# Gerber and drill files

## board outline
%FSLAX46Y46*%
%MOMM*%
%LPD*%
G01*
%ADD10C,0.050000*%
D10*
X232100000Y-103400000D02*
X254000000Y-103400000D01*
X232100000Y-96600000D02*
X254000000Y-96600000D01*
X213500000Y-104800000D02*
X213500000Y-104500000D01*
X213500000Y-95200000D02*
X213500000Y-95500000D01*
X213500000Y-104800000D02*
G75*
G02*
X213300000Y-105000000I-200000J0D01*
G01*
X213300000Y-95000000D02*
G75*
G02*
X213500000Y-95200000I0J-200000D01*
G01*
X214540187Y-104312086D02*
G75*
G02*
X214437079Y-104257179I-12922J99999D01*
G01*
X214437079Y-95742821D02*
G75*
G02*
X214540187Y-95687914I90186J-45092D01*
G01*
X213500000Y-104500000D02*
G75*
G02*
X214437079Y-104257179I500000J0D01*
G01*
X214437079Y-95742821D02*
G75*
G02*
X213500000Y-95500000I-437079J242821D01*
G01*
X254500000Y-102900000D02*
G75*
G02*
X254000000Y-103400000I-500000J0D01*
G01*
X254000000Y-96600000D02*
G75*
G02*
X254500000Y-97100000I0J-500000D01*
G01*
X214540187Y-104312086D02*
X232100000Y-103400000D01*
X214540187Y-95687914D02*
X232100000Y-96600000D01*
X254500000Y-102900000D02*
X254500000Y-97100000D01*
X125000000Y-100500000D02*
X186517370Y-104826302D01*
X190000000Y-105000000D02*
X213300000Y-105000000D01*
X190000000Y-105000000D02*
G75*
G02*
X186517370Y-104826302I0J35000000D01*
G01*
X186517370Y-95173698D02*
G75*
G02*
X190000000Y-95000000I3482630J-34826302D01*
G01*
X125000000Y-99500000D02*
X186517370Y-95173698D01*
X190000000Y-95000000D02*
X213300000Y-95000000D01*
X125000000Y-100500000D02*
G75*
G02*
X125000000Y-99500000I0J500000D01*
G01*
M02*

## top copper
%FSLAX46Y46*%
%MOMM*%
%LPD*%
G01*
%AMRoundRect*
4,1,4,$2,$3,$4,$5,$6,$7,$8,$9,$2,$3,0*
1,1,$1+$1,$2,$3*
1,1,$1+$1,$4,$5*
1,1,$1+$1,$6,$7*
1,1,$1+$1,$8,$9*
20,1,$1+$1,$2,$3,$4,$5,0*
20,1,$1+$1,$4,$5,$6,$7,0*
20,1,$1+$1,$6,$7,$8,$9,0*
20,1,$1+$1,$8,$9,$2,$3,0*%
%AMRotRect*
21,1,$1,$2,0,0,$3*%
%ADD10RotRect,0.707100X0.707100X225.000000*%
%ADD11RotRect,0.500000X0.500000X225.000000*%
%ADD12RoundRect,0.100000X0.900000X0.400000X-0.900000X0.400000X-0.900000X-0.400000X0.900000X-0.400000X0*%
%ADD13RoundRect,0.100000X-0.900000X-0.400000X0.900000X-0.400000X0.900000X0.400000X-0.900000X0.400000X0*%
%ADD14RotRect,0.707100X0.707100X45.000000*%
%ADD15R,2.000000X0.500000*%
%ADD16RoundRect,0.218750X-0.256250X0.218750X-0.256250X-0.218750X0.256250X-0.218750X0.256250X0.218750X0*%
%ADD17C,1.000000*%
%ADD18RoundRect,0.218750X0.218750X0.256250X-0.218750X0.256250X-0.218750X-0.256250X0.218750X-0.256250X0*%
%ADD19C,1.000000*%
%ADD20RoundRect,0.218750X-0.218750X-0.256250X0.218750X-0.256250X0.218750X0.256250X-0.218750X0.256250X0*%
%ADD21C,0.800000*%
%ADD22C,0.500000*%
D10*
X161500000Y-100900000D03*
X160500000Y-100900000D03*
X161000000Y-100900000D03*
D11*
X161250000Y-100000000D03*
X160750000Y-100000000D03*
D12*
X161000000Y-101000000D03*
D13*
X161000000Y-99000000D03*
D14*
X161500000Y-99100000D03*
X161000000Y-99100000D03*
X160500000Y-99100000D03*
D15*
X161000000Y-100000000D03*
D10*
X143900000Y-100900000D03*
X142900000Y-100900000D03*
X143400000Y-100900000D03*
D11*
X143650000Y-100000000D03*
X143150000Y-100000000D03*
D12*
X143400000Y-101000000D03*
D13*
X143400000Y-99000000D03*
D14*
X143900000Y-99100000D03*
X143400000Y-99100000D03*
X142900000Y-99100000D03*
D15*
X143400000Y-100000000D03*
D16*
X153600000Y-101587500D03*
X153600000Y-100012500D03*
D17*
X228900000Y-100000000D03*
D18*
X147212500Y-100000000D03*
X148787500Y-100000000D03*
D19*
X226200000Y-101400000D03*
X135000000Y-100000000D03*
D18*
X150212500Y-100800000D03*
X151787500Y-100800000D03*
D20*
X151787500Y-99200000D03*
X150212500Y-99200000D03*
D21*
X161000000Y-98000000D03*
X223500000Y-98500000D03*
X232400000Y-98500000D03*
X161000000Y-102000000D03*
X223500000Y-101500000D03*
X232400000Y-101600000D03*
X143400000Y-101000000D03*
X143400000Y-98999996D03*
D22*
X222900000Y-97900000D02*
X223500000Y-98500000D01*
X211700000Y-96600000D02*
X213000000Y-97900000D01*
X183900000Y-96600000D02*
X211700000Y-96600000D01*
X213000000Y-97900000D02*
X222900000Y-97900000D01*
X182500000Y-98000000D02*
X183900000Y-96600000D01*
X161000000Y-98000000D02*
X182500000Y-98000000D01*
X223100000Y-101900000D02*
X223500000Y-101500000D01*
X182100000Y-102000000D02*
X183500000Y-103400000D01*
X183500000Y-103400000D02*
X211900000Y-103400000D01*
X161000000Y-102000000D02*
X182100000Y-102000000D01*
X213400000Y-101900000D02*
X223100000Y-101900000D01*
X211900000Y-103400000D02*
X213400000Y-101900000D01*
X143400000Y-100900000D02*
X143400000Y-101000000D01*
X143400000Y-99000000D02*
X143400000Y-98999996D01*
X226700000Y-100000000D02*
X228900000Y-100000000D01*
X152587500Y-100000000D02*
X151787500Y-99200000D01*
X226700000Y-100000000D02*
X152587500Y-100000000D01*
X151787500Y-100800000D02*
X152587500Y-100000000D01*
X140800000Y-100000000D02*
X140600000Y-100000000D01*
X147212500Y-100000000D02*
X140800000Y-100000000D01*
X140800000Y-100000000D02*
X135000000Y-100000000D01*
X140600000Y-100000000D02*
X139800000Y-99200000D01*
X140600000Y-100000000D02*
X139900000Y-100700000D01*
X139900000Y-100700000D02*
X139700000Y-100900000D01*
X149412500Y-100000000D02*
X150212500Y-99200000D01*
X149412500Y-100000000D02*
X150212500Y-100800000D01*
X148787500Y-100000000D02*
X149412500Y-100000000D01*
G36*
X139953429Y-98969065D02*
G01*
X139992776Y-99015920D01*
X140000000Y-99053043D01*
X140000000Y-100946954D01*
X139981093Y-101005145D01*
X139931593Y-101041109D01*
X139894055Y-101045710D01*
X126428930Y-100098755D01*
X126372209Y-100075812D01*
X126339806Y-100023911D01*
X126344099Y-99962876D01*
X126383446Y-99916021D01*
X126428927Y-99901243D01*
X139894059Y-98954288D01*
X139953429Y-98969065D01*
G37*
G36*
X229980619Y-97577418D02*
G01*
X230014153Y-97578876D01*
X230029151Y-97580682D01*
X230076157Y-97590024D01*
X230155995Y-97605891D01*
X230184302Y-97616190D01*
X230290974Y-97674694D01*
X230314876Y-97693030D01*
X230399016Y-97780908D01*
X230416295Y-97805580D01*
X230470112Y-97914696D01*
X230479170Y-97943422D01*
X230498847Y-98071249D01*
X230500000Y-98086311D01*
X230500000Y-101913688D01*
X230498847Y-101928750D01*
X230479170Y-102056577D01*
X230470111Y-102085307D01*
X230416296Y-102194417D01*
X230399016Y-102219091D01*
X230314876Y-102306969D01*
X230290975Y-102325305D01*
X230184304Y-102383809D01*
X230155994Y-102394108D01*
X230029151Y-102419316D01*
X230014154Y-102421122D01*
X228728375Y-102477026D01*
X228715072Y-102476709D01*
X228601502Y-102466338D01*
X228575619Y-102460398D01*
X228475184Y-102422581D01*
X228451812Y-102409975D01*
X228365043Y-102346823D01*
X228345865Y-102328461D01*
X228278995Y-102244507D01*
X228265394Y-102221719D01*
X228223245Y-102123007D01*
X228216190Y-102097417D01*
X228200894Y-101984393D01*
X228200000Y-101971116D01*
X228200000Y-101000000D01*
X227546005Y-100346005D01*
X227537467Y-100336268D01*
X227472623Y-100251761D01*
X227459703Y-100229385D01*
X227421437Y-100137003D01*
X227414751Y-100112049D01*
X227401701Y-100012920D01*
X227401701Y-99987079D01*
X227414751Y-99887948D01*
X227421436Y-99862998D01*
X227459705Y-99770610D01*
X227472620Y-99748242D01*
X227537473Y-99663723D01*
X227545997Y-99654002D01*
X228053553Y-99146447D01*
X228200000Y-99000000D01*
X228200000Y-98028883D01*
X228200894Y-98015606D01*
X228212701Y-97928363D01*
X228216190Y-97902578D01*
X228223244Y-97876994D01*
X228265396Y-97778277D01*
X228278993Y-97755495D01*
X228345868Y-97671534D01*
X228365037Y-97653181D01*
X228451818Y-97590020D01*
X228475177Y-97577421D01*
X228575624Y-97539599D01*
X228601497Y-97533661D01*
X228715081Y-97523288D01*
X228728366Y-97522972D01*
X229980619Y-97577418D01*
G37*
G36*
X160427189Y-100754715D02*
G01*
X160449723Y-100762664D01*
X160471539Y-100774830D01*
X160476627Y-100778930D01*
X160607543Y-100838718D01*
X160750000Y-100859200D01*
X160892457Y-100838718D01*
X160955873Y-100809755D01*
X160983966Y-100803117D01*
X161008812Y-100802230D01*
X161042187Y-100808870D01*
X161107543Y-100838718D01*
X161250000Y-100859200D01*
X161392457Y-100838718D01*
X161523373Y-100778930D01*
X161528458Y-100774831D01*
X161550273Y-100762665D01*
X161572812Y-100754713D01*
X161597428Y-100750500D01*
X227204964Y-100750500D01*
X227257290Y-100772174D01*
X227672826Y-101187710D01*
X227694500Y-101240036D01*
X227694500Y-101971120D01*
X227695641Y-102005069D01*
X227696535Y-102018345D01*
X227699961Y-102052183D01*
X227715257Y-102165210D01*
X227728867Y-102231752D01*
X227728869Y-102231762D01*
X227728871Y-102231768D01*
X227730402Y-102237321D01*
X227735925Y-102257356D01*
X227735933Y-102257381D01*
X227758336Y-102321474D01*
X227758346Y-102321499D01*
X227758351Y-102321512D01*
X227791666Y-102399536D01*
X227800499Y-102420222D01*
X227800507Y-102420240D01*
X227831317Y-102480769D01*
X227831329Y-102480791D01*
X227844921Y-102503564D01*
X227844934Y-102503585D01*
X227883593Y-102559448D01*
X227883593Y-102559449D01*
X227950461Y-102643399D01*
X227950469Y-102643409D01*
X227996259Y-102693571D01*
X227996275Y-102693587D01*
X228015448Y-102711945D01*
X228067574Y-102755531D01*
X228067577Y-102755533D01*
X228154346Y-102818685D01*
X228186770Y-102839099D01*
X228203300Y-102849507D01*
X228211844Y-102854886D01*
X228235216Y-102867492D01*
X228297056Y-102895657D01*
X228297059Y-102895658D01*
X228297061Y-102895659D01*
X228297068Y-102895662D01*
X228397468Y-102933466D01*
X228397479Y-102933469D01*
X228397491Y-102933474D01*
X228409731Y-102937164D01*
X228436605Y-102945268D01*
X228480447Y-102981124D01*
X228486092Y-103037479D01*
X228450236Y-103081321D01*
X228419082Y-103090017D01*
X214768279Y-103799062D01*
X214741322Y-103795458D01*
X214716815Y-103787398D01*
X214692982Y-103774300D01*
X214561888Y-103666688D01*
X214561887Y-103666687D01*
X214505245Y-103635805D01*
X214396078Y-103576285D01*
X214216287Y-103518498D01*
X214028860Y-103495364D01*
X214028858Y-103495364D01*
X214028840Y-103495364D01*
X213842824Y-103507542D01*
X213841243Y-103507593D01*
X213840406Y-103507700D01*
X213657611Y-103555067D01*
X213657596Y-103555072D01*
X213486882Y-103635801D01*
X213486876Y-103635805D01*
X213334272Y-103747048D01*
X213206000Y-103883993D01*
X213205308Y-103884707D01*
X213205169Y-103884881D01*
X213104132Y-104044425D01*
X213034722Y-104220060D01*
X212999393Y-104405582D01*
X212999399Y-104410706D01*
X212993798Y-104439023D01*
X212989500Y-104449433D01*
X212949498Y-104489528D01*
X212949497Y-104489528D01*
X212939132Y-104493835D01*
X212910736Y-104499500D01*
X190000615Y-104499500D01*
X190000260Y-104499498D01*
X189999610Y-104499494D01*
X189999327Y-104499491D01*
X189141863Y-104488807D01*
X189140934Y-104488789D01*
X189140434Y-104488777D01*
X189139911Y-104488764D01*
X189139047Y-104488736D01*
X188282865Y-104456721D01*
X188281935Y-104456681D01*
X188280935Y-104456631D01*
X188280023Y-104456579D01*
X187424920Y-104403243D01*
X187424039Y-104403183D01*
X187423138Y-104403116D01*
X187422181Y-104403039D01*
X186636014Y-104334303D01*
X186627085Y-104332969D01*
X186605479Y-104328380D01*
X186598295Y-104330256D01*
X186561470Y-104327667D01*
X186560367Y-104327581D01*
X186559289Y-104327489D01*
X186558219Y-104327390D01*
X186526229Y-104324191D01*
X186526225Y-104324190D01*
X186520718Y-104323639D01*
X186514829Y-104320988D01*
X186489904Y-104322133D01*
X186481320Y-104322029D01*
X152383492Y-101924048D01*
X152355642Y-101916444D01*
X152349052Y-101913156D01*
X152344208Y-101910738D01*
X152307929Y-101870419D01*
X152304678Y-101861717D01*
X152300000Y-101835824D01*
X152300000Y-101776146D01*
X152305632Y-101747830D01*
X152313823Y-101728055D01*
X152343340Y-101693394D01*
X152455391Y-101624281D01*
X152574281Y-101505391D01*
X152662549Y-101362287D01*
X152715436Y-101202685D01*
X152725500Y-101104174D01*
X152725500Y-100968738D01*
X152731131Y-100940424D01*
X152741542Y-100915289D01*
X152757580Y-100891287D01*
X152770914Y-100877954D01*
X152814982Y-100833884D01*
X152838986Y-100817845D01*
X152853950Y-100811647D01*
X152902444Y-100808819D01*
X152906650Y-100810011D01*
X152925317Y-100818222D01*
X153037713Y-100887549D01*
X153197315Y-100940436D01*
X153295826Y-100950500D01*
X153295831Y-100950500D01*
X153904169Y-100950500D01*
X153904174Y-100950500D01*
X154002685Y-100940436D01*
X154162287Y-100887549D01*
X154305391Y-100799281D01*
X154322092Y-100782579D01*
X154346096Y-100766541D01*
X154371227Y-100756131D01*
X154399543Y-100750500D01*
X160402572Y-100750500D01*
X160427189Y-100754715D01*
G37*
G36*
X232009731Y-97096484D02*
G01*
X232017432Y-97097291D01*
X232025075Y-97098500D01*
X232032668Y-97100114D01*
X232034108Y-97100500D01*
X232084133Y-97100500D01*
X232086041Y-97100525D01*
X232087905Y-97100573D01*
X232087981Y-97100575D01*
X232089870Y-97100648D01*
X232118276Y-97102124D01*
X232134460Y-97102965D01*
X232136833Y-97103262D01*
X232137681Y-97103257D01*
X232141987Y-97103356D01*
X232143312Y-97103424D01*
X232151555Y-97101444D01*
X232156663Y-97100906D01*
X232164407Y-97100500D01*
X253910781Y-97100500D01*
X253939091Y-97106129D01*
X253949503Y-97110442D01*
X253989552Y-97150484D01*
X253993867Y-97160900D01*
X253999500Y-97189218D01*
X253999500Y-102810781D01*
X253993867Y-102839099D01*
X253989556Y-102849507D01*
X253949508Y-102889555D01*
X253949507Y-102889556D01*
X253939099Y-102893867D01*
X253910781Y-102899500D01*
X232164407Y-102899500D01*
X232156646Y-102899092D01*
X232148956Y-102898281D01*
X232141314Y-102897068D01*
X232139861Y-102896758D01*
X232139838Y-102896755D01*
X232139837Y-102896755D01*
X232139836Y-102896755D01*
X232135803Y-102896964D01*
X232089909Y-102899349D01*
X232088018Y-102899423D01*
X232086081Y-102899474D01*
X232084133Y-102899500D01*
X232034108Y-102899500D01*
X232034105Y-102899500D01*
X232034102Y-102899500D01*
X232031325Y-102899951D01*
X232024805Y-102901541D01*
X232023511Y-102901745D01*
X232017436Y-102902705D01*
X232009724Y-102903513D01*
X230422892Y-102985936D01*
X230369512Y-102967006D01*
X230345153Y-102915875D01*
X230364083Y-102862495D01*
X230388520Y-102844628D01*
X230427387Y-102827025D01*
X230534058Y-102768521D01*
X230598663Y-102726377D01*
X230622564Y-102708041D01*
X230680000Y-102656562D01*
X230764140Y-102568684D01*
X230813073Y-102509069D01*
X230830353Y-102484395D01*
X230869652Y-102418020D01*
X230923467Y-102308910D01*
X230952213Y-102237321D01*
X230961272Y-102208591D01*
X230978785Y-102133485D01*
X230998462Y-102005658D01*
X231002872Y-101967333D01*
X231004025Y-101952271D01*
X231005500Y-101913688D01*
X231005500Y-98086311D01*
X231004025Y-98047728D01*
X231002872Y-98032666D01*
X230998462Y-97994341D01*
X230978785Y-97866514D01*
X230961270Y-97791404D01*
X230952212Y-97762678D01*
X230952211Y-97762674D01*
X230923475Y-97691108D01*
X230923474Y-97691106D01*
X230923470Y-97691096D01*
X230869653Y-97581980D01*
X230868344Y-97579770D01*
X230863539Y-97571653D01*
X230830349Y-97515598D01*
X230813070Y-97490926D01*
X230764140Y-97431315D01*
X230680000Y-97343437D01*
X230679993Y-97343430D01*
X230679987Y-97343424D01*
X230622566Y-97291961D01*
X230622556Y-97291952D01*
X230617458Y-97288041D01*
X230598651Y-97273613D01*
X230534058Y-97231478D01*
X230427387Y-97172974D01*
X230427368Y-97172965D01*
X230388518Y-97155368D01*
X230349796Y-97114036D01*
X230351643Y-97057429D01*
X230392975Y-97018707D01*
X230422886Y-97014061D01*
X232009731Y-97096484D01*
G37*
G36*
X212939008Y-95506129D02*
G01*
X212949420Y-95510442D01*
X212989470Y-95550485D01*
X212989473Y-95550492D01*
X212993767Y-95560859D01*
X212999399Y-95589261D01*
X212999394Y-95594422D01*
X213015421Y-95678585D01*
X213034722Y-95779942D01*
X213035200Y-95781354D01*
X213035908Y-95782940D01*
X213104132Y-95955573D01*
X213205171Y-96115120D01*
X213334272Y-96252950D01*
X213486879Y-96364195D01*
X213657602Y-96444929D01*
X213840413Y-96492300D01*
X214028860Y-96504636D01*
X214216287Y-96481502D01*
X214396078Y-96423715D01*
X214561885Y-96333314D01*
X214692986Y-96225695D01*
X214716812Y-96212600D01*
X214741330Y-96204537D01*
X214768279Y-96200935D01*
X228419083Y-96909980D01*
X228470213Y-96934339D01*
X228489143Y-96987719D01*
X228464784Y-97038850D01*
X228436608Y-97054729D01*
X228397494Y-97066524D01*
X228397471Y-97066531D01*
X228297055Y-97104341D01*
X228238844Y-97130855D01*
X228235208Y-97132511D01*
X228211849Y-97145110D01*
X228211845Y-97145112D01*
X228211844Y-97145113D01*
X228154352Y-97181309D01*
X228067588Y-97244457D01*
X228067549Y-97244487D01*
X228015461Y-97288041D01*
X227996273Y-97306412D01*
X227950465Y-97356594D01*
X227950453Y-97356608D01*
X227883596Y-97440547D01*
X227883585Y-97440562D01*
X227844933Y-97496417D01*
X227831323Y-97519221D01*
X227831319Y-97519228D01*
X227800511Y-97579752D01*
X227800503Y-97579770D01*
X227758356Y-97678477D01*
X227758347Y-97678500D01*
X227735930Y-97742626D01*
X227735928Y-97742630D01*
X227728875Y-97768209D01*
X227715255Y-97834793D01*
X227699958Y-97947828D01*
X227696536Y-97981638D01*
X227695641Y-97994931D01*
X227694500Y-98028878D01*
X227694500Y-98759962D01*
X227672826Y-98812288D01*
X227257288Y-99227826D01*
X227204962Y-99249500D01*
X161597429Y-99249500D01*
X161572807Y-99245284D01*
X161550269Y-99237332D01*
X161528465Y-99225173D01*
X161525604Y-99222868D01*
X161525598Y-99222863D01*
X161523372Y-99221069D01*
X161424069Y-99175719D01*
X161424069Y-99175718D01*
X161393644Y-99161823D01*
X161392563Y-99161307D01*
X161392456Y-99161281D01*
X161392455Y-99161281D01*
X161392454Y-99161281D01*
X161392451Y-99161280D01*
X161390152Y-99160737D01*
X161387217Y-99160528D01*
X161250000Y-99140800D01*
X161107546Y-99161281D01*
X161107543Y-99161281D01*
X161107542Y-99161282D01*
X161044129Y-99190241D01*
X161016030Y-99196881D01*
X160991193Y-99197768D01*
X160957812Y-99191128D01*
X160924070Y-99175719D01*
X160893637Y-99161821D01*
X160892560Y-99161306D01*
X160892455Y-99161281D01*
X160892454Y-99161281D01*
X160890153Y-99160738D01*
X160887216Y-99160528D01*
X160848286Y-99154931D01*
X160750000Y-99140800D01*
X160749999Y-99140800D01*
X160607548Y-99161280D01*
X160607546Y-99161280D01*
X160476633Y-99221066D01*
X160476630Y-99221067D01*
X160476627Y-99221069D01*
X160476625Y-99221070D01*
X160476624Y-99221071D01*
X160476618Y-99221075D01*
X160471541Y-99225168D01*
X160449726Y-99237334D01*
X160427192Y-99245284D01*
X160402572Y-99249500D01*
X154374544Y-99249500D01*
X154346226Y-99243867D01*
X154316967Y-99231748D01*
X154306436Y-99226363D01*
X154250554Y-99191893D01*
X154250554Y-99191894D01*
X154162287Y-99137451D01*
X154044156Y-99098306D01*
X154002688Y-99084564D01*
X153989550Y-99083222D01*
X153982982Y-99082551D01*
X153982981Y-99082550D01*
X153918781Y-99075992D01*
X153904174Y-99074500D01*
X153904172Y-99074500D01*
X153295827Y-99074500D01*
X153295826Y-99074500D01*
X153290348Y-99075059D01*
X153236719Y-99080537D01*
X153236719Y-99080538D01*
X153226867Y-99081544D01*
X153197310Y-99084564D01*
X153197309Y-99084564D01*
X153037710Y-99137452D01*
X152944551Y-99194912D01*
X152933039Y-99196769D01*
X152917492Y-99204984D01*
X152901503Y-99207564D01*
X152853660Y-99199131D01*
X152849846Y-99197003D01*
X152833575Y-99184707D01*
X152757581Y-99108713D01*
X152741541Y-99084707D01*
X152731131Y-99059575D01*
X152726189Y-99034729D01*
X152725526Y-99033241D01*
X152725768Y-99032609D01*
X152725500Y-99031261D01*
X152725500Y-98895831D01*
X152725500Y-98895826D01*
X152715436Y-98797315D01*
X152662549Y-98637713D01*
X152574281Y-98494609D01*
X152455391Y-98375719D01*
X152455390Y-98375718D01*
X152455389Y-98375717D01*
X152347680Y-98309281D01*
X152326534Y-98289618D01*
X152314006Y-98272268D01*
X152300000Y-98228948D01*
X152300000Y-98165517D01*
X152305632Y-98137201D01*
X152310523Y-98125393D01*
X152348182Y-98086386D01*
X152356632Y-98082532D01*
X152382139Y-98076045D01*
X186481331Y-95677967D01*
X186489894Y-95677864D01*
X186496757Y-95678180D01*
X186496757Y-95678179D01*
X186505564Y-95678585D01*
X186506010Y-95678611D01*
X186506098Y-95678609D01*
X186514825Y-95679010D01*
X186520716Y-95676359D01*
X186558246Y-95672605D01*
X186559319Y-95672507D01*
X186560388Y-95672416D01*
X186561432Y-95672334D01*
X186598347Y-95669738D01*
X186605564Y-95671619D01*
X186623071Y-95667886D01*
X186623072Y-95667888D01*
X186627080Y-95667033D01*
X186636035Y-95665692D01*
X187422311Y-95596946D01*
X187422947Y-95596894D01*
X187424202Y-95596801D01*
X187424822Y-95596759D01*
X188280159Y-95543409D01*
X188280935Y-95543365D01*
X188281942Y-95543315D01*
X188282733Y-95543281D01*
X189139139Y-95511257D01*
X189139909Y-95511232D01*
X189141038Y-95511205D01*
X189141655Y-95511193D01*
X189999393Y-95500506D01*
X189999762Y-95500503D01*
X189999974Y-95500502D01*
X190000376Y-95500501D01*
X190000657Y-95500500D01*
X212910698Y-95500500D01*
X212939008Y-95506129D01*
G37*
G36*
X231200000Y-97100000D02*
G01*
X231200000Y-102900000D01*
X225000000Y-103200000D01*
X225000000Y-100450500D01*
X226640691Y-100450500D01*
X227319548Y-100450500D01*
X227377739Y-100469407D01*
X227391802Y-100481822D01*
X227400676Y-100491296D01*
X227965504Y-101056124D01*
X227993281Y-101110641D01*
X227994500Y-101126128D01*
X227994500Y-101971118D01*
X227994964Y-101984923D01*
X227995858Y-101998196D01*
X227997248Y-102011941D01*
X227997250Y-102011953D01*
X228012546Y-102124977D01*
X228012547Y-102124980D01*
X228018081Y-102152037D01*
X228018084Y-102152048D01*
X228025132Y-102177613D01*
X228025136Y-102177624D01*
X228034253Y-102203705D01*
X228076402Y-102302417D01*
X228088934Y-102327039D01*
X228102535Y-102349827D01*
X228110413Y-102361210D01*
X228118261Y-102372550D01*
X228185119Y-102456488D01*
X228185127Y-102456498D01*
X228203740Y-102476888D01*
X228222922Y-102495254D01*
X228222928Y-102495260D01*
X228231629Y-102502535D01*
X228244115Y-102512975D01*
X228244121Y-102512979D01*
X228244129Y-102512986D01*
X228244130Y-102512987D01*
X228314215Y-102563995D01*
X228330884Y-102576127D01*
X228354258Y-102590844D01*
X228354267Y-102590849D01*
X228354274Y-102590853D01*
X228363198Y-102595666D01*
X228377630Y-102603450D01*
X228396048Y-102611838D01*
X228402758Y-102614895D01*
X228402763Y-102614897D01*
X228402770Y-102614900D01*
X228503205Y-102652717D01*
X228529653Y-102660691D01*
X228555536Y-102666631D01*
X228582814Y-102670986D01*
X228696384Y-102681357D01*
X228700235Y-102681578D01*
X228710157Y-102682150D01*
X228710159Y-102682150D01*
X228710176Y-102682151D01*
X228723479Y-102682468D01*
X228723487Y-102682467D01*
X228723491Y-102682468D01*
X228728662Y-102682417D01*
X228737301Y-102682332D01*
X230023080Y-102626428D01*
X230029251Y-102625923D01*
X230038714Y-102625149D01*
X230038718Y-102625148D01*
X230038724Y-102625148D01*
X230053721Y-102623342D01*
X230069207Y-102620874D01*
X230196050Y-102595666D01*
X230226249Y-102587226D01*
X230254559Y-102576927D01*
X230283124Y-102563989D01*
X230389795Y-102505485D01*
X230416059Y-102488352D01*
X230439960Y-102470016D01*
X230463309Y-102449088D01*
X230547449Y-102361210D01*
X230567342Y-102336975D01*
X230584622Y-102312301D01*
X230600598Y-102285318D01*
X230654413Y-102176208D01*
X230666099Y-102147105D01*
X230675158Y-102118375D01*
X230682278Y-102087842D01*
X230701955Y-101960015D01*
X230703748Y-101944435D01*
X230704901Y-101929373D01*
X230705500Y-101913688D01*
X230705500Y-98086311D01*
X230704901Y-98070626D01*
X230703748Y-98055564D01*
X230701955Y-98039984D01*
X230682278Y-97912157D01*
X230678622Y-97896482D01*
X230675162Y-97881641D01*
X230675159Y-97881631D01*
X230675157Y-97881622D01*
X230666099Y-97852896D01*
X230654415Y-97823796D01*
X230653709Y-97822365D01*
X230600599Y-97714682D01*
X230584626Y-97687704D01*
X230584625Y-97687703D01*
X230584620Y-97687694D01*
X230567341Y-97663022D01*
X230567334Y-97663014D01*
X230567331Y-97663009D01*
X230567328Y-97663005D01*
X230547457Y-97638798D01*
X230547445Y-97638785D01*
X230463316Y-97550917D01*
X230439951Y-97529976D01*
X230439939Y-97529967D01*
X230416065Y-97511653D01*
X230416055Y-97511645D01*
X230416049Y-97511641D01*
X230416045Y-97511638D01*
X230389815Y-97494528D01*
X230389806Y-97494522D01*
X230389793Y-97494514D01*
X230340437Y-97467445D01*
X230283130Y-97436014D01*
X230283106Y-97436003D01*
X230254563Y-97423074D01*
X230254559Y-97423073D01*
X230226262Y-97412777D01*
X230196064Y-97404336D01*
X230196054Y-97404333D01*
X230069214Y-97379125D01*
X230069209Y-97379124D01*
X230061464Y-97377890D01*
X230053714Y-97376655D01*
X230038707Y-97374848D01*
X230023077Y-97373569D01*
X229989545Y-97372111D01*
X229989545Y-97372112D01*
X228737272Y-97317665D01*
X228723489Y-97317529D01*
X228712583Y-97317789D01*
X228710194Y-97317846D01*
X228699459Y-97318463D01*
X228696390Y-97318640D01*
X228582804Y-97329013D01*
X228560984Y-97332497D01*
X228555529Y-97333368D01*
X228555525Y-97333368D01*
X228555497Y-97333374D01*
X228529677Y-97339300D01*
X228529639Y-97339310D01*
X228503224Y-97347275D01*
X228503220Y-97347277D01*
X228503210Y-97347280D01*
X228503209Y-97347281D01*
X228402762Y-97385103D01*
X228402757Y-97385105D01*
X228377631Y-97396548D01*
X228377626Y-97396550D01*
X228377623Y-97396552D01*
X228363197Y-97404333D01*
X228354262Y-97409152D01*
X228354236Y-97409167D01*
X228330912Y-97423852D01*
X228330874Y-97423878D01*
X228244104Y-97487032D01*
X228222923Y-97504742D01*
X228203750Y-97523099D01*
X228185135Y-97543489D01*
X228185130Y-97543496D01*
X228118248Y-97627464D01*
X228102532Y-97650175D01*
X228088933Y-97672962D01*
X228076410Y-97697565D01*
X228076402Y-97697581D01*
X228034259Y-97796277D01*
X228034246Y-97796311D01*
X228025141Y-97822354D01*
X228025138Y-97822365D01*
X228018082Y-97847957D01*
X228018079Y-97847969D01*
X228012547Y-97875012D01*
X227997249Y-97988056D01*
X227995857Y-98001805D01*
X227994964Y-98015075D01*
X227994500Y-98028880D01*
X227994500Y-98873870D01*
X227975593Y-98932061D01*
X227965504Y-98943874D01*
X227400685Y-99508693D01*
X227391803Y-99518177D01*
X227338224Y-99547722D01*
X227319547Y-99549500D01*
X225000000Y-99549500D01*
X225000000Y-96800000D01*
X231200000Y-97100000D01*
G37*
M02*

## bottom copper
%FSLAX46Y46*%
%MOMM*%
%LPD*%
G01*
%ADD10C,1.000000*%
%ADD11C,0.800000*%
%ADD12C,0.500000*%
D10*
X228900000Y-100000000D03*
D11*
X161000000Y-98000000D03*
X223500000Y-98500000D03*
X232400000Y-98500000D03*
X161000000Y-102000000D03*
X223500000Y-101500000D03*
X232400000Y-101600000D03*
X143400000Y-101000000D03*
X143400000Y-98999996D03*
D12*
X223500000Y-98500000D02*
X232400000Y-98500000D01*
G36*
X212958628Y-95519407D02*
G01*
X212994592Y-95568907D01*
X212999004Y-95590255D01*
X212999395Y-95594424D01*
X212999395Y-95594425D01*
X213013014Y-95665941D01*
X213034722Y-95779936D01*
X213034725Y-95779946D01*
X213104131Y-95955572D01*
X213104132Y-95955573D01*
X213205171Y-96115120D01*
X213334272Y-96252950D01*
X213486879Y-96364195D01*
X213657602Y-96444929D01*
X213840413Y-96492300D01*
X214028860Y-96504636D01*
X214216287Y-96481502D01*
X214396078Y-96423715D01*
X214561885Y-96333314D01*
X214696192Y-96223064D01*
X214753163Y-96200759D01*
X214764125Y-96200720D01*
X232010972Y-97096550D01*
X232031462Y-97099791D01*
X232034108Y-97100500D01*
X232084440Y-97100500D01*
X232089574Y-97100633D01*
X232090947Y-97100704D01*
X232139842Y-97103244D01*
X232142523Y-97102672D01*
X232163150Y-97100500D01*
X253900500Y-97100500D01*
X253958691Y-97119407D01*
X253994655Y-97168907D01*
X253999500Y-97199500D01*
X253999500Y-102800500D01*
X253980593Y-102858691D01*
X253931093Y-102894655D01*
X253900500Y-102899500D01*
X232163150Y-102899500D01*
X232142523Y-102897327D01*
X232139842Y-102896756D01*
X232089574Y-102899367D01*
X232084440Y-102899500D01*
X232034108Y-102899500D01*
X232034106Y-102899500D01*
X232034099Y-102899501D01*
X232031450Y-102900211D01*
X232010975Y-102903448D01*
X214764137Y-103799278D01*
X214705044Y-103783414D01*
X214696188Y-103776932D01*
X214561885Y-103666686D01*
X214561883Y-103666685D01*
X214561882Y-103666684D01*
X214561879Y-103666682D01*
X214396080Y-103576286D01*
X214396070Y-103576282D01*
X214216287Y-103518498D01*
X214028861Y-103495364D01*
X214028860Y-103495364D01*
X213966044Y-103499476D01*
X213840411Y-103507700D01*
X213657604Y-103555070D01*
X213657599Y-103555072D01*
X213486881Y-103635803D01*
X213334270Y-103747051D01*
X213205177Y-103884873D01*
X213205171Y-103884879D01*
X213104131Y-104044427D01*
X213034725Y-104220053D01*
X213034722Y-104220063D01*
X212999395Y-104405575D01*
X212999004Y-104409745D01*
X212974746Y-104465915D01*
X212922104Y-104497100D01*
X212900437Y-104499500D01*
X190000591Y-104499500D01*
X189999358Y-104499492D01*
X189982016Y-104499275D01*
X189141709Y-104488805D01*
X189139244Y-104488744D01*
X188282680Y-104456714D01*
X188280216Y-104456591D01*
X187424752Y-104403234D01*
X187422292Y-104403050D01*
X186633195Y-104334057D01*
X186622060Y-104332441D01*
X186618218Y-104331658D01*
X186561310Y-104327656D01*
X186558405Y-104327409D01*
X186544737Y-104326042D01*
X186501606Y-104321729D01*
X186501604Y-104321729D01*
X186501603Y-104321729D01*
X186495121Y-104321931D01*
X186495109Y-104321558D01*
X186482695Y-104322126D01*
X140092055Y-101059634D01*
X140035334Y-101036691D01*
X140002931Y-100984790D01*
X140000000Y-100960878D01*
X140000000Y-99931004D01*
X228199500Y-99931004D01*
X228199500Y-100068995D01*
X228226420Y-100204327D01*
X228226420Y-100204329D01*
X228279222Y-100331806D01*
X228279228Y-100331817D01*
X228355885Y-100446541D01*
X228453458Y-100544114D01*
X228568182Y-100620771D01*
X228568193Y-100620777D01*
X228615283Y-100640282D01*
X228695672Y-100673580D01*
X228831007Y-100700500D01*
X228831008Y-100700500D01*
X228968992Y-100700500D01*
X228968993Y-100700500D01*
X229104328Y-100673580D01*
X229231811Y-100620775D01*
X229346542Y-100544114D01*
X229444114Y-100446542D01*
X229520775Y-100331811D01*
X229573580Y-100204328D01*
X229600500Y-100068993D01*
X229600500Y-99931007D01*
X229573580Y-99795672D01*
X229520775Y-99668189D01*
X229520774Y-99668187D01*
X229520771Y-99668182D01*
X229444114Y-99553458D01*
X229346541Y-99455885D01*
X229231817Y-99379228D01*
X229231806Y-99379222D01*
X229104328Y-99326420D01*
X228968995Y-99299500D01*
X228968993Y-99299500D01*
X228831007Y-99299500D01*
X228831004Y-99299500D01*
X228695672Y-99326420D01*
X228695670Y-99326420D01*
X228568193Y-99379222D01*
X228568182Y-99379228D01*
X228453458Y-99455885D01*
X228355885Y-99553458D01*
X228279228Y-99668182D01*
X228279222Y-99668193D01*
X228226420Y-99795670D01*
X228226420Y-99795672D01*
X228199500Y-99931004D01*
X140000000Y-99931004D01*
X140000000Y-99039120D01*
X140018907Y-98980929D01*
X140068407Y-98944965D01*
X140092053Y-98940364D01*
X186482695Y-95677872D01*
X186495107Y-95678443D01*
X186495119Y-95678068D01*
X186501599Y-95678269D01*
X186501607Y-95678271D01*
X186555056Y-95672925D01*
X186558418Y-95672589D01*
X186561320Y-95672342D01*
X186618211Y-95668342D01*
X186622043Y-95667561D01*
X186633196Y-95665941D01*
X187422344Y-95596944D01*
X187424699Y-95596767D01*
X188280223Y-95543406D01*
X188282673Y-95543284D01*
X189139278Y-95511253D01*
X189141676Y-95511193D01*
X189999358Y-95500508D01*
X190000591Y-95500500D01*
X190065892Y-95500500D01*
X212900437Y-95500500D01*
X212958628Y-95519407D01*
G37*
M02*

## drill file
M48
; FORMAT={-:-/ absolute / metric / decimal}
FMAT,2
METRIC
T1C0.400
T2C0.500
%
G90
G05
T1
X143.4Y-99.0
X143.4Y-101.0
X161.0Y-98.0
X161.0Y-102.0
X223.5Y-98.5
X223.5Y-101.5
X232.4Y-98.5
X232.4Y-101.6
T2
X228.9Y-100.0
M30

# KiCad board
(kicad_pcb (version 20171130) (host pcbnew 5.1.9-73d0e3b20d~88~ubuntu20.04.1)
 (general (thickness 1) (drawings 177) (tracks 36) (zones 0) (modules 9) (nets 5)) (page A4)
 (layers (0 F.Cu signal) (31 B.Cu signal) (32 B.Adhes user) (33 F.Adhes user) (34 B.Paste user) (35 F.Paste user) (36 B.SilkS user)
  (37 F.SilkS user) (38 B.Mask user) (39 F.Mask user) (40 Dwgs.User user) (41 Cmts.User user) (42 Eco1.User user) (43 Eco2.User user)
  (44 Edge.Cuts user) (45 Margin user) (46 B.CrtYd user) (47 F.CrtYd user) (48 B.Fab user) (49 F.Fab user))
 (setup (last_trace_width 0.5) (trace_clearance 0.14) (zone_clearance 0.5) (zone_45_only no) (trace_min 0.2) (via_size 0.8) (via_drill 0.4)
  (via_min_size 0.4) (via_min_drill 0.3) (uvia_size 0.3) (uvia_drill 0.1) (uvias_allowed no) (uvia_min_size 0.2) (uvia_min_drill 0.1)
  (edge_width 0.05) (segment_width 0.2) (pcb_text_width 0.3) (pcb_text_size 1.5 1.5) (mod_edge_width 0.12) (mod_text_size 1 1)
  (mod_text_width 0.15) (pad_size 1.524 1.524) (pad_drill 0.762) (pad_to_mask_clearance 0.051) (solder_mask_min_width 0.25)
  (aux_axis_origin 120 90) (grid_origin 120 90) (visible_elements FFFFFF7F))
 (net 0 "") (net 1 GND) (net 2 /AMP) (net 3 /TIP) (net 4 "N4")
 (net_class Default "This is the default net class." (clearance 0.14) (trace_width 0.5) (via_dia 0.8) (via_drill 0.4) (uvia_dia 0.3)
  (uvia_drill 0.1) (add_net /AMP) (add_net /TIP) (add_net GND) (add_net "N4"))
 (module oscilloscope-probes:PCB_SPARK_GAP (layer F.Cu) (at 161 100)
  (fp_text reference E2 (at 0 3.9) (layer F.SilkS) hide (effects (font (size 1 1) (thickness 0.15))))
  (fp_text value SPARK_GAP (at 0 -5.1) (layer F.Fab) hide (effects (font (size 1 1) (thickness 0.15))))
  (pad 2 smd rect (at 0.5 0.9 225) (size 0.7071 0.7071) (layers F.Cu) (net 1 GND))
  (pad 2 smd rect (at -0.5 0.9 225) (size 0.7071 0.7071) (layers F.Cu) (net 1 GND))
  (pad 2 smd rect (at 0 0.9 225) (size 0.7071 0.7071) (layers F.Cu) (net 1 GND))
  (pad 1 smd rect (at 0.25 0 225) (size 0.5 0.5) (layers F.Cu F.Mask) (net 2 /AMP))
  (pad 1 smd rect (at -0.25 0 225) (size 0.5 0.5) (layers F.Cu F.Mask) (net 2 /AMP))
  (pad 2 smd roundrect (at 0 1 180) (size 2 1) (layers F.Cu) (roundrect_rratio 0.1) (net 1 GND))
  (pad 2 smd roundrect (at 0 -1) (size 2 1) (layers F.Cu) (roundrect_rratio 0.1) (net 1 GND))
  (pad 2 smd rect (at 0.5 -0.9 45) (size 0.7071 0.7071) (layers F.Cu) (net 1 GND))
  (pad 2 smd rect (at 0 -0.9 45) (size 0.7071 0.7071) (layers F.Cu) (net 1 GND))
  (pad 2 smd rect (at -0.5 -0.9 45) (size 0.7071 0.7071) (layers F.Cu) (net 1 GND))
  (pad 1 smd rect (at 0 0) (size 2 0.5) (layers F.Cu F.Mask) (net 2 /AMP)))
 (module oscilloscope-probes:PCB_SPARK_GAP (layer F.Cu) (at 143.4 100)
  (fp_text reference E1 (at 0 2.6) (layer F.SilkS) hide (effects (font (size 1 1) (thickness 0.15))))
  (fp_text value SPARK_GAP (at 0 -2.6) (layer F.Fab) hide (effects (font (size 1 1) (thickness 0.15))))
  (pad 2 smd rect (at 0.5 0.9 225) (size 0.7071 0.7071) (layers F.Cu) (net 1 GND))
  (pad 2 smd rect (at -0.5 0.9 225) (size 0.7071 0.7071) (layers F.Cu) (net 1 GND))
  (pad 2 smd rect (at 0 0.9 225) (size 0.7071 0.7071) (layers F.Cu) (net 1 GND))
  (pad 1 smd rect (at 0.25 0 225) (size 0.5 0.5) (layers F.Cu F.Mask) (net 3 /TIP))
  (pad 1 smd rect (at -0.25 0 225) (size 0.5 0.5) (layers F.Cu F.Mask) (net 3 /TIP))
  (pad 2 smd roundrect (at 0 1 180) (size 2 1) (layers F.Cu) (roundrect_rratio 0.1) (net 1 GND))
  (pad 2 smd roundrect (at 0 -1) (size 2 1) (layers F.Cu) (roundrect_rratio 0.1) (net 1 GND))
  (pad 2 smd rect (at 0.5 -0.9 45) (size 0.7071 0.7071) (layers F.Cu) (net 1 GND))
  (pad 2 smd rect (at 0 -0.9 45) (size 0.7071 0.7071) (layers F.Cu) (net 1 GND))
  (pad 2 smd rect (at -0.5 -0.9 45) (size 0.7071 0.7071) (layers F.Cu) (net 1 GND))
  (pad 1 smd rect (at 0 0) (size 2 0.5) (layers F.Cu F.Mask) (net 3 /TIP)))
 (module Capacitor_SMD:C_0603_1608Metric (layer F.Cu) (at 153.6 100.8 270)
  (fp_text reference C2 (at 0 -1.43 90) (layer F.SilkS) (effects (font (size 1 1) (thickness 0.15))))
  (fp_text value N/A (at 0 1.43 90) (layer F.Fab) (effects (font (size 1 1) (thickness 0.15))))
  (pad 2 smd roundrect (at 0.7875 0 270) (size 0.875 0.95) (layers F.Cu F.Paste F.Mask) (roundrect_rratio 0.25) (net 1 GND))
  (pad 1 smd roundrect (at -0.7875 0 270) (size 0.875 0.95) (layers F.Cu F.Paste F.Mask) (roundrect_rratio 0.25) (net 2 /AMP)))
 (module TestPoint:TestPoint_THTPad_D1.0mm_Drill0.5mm (layer F.Cu) (at 228.9 100)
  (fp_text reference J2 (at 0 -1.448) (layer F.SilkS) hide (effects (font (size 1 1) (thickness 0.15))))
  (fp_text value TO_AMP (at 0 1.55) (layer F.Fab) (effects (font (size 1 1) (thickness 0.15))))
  (pad 1 thru_hole circle (at 0 0) (size 1 1) (drill 0.5) (layers *.Cu *.Mask) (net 2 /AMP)))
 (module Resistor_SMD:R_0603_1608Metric (layer F.Cu) (at 148 100 180)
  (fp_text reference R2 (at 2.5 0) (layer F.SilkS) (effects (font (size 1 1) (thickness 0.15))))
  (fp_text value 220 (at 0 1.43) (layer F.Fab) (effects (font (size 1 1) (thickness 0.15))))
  (pad 2 smd roundrect (at 0.7875 0 180) (size 0.875 0.95) (layers F.Cu F.Paste F.Mask) (roundrect_rratio 0.25) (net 3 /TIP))
  (pad 1 smd roundrect (at -0.7875 0 180) (size 0.875 0.95) (layers F.Cu F.Paste F.Mask) (roundrect_rratio 0.25) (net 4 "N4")))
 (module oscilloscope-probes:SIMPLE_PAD (layer F.Cu) (at 226.2 101.4)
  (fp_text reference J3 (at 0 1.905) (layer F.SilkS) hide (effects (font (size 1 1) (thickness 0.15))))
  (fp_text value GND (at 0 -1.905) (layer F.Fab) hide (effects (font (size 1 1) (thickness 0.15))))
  (pad 1 smd circle (at 0 0) (size 1 1) (layers F.Cu F.Mask) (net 1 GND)))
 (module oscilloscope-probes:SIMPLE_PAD (layer F.Cu) (at 135 100)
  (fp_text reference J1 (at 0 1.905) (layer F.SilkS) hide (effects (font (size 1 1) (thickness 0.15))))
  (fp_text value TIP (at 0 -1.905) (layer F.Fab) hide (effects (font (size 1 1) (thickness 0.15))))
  (pad 1 smd circle (at 0 0) (size 1 1) (layers F.Cu F.Mask) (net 3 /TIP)))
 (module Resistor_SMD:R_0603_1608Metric (layer F.Cu) (at 151 100.8 180)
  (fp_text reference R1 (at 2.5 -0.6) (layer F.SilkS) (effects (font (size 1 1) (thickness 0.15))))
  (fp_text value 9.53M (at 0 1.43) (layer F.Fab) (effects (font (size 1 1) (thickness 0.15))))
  (pad 2 smd roundrect (at 0.7875 0 180) (size 0.875 0.95) (layers F.Cu F.Paste F.Mask) (roundrect_rratio 0.25) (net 4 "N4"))
  (pad 1 smd roundrect (at -0.7875 0 180) (size 0.875 0.95) (layers F.Cu F.Paste F.Mask) (roundrect_rratio 0.25) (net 2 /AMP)))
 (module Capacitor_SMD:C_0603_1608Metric (layer F.Cu) (at 151 99.2)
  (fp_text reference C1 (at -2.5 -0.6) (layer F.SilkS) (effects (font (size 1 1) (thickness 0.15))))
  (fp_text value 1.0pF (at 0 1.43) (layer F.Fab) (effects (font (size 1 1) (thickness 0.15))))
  (pad 2 smd roundrect (at 0.7875 0) (size 0.875 0.95) (layers F.Cu F.Paste F.Mask) (roundrect_rratio 0.25) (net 2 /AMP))
  (pad 1 smd roundrect (at -0.7875 0) (size 0.875 0.95) (layers F.Cu F.Paste F.Mask) (roundrect_rratio 0.25) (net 4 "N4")))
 (gr_line (start 232.1 103.4) (end 254 103.4) (layer Edge.Cuts) (width 0.05))
 (gr_line (start 232.1 96.6) (end 254 96.6) (layer Edge.Cuts) (width 0.05))
 (gr_line (start 213.5 104.8) (end 213.5 104.5) (layer Edge.Cuts) (width 0.05))
 (gr_line (start 213.5 95.2) (end 213.5 95.5) (layer Edge.Cuts) (width 0.05))
 (gr_arc (start 213.3 104.8) (end 213.5 104.8) (angle 90) (layer Edge.Cuts) (width 0.05))
 (gr_arc (start 213.3 95.2) (end 213.5 95.2) (angle -90) (layer Edge.Cuts) (width 0.05))
 (gr_arc (start 214.527265 104.212087) (end 214.540187 104.312086) (angle 70.79848966) (layer Edge.Cuts) (width 0.05))
 (gr_arc (start 214.527265 95.787913) (end 214.540187 95.687914) (angle -70.79848966) (layer Edge.Cuts) (width 0.05))
 (gr_arc (start 214 104.5) (end 213.5 104.5) (angle 150.9453959) (layer Edge.Cuts) (width 0.05))
 (gr_arc (start 214 95.5) (end 213.5 95.5) (angle -150.9453959) (layer Edge.Cuts) (width 0.05))
 (gr_arc (start 254 102.9) (end 254 103.4) (angle -90) (layer Edge.Cuts) (width 0.05))
 (gr_arc (start 254 97.1) (end 254.5 97.1) (angle -90) (layer Edge.Cuts) (width 0.05))
 (gr_line (start 214.540187 104.312086) (end 232.1 103.4) (layer Edge.Cuts) (width 0.05))
 (gr_line (start 214.540187 95.687914) (end 232.1 96.6) (layer Edge.Cuts) (width 0.05))
 (gr_line (start 254.5 102.9) (end 254.5 97.1) (layer Edge.Cuts) (width 0.05))
 (gr_line (start 125 100.5) (end 186.51737 104.826302) (layer Edge.Cuts) (width 0.05))
 (gr_line (start 190 105) (end 213.3 105) (layer Edge.Cuts) (width 0.05))
 (gr_arc (start 190 70) (end 190 105) (angle 5.710593137) (layer Edge.Cuts) (width 0.05))
 (gr_arc (start 190 130) (end 190 95) (angle -5.710593137) (layer Edge.Cuts) (width 0.05))
 (gr_line (start 125 99.5) (end 186.51737 95.173698) (layer Edge.Cuts) (width 0.05))
 (gr_line (start 190 95) (end 213.3 95) (layer Edge.Cuts) (width 0.05))
 (gr_arc (start 125 100) (end 125 99.5) (angle -180) (layer Edge.Cuts) (width 0.05))
 (via (at 161 98) (size 0.8) (drill 0.4) (layers F.Cu B.Cu) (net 1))
 (via (at 223.5 98.5) (size 0.8) (drill 0.4) (layers F.Cu B.Cu) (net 1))
 (segment (start 222.9 97.9) (end 223.5 98.5) (width 0.5) (layer F.Cu) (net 1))
 (segment (start 211.7 96.6) (end 213 97.9) (width 0.5) (layer F.Cu) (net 1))
 (segment (start 183.9 96.6) (end 211.7 96.6) (width 0.5) (layer F.Cu) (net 1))
 (segment (start 213 97.9) (end 222.9 97.9) (width 0.5) (layer F.Cu) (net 1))
 (segment (start 182.5 98) (end 183.9 96.6) (width 0.5) (layer F.Cu) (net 1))
 (segment (start 161 98) (end 182.5 98) (width 0.5) (layer F.Cu) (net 1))
 (via (at 232.4 98.5) (size 0.8) (drill 0.4) (layers F.Cu B.Cu) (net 1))
 (segment (start 223.5 98.5) (end 232.4 98.5) (width 0.5) (layer B.Cu) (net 1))
 (via (at 161 102) (size 0.8) (drill 0.4) (layers F.Cu B.Cu) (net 1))
 (segment (start 223.1 101.9) (end 223.5 101.5) (width 0.5) (layer F.Cu) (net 1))
 (via (at 223.5 101.5) (size 0.8) (drill 0.4) (layers F.Cu B.Cu) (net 1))
 (segment (start 182.1 102) (end 183.5 103.4) (width 0.5) (layer F.Cu) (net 1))
 (via (at 232.4 101.6) (size 0.8) (drill 0.4) (layers F.Cu B.Cu) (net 1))
 (segment (start 183.5 103.4) (end 211.9 103.4) (width 0.5) (layer F.Cu) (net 1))
 (segment (start 161 102) (end 182.1 102) (width 0.5) (layer F.Cu) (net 1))
 (segment (start 213.4 101.9) (end 223.1 101.9) (width 0.5) (layer F.Cu) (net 1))
 (segment (start 211.9 103.4) (end 213.4 101.9) (width 0.5) (layer F.Cu) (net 1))
 (via (at 143.4 101) (size 0.8) (drill 0.4) (layers F.Cu B.Cu) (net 1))
 (segment (start 143.4 100.9) (end 143.4 101) (width 0.5) (layer F.Cu) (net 1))
 (via (at 143.4 98.999996) (size 0.8) (drill 0.4) (layers F.Cu B.Cu) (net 1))
 (segment (start 143.4 99) (end 143.4 98.999996) (width 0.5) (layer F.Cu) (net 1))
 (segment (start 226.7 100) (end 228.9 100) (width 0.5) (layer F.Cu) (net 2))
 (segment (start 152.5875 100) (end 151.7875 99.2) (width 0.5) (layer F.Cu) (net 2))
 (segment (start 226.7 100) (end 152.5875 100) (width 0.5) (layer F.Cu) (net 2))
 (segment (start 151.7875 100.8) (end 152.5875 100) (width 0.5) (layer F.Cu) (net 2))
 (segment (start 140.8 100) (end 140.6 100) (width 0.5) (layer F.Cu) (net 3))
 (segment (start 147.2125 100) (end 140.8 100) (width 0.5) (layer F.Cu) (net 3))
 (segment (start 140.8 100) (end 135 100) (width 0.5) (layer F.Cu) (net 3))
 (segment (start 140.6 100) (end 139.8 99.2) (width 0.5) (layer F.Cu) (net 3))
 (segment (start 140.6 100) (end 139.9 100.7) (width 0.5) (layer F.Cu) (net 3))
 (segment (start 139.9 100.7) (end 139.7 100.9) (width 0.5) (layer F.Cu) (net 3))
 (segment (start 149.4125 100) (end 150.2125 99.2) (width 0.5) (layer F.Cu) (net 4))
 (segment (start 149.4125 100) (end 150.2125 100.8) (width 0.5) (layer F.Cu) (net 4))
 (segment (start 148.7875 100) (end 149.4125 100) (width 0.5) (layer F.Cu) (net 4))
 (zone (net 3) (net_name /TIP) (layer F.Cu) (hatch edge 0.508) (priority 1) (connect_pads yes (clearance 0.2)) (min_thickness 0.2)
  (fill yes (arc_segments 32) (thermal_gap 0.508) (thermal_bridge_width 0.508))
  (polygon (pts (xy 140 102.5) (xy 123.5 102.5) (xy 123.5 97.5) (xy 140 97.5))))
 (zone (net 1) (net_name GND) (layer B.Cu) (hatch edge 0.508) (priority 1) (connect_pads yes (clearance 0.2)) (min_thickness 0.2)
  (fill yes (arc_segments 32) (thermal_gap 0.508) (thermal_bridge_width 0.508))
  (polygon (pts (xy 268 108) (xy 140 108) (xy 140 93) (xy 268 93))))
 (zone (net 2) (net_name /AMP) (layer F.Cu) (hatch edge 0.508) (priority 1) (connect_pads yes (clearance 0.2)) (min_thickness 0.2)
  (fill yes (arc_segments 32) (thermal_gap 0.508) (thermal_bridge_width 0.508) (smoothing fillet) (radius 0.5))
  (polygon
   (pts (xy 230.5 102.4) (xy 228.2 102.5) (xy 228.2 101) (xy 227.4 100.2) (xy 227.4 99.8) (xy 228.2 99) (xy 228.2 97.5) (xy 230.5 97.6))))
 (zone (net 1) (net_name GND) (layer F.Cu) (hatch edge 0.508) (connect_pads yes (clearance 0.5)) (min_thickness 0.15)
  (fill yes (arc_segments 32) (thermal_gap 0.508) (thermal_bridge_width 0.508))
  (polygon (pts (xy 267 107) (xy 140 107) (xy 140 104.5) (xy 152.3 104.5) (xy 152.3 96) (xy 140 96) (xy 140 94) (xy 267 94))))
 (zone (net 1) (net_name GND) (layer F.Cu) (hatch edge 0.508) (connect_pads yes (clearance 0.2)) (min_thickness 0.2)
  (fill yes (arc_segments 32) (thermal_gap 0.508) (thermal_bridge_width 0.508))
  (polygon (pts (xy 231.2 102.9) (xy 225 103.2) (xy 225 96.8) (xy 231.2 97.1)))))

